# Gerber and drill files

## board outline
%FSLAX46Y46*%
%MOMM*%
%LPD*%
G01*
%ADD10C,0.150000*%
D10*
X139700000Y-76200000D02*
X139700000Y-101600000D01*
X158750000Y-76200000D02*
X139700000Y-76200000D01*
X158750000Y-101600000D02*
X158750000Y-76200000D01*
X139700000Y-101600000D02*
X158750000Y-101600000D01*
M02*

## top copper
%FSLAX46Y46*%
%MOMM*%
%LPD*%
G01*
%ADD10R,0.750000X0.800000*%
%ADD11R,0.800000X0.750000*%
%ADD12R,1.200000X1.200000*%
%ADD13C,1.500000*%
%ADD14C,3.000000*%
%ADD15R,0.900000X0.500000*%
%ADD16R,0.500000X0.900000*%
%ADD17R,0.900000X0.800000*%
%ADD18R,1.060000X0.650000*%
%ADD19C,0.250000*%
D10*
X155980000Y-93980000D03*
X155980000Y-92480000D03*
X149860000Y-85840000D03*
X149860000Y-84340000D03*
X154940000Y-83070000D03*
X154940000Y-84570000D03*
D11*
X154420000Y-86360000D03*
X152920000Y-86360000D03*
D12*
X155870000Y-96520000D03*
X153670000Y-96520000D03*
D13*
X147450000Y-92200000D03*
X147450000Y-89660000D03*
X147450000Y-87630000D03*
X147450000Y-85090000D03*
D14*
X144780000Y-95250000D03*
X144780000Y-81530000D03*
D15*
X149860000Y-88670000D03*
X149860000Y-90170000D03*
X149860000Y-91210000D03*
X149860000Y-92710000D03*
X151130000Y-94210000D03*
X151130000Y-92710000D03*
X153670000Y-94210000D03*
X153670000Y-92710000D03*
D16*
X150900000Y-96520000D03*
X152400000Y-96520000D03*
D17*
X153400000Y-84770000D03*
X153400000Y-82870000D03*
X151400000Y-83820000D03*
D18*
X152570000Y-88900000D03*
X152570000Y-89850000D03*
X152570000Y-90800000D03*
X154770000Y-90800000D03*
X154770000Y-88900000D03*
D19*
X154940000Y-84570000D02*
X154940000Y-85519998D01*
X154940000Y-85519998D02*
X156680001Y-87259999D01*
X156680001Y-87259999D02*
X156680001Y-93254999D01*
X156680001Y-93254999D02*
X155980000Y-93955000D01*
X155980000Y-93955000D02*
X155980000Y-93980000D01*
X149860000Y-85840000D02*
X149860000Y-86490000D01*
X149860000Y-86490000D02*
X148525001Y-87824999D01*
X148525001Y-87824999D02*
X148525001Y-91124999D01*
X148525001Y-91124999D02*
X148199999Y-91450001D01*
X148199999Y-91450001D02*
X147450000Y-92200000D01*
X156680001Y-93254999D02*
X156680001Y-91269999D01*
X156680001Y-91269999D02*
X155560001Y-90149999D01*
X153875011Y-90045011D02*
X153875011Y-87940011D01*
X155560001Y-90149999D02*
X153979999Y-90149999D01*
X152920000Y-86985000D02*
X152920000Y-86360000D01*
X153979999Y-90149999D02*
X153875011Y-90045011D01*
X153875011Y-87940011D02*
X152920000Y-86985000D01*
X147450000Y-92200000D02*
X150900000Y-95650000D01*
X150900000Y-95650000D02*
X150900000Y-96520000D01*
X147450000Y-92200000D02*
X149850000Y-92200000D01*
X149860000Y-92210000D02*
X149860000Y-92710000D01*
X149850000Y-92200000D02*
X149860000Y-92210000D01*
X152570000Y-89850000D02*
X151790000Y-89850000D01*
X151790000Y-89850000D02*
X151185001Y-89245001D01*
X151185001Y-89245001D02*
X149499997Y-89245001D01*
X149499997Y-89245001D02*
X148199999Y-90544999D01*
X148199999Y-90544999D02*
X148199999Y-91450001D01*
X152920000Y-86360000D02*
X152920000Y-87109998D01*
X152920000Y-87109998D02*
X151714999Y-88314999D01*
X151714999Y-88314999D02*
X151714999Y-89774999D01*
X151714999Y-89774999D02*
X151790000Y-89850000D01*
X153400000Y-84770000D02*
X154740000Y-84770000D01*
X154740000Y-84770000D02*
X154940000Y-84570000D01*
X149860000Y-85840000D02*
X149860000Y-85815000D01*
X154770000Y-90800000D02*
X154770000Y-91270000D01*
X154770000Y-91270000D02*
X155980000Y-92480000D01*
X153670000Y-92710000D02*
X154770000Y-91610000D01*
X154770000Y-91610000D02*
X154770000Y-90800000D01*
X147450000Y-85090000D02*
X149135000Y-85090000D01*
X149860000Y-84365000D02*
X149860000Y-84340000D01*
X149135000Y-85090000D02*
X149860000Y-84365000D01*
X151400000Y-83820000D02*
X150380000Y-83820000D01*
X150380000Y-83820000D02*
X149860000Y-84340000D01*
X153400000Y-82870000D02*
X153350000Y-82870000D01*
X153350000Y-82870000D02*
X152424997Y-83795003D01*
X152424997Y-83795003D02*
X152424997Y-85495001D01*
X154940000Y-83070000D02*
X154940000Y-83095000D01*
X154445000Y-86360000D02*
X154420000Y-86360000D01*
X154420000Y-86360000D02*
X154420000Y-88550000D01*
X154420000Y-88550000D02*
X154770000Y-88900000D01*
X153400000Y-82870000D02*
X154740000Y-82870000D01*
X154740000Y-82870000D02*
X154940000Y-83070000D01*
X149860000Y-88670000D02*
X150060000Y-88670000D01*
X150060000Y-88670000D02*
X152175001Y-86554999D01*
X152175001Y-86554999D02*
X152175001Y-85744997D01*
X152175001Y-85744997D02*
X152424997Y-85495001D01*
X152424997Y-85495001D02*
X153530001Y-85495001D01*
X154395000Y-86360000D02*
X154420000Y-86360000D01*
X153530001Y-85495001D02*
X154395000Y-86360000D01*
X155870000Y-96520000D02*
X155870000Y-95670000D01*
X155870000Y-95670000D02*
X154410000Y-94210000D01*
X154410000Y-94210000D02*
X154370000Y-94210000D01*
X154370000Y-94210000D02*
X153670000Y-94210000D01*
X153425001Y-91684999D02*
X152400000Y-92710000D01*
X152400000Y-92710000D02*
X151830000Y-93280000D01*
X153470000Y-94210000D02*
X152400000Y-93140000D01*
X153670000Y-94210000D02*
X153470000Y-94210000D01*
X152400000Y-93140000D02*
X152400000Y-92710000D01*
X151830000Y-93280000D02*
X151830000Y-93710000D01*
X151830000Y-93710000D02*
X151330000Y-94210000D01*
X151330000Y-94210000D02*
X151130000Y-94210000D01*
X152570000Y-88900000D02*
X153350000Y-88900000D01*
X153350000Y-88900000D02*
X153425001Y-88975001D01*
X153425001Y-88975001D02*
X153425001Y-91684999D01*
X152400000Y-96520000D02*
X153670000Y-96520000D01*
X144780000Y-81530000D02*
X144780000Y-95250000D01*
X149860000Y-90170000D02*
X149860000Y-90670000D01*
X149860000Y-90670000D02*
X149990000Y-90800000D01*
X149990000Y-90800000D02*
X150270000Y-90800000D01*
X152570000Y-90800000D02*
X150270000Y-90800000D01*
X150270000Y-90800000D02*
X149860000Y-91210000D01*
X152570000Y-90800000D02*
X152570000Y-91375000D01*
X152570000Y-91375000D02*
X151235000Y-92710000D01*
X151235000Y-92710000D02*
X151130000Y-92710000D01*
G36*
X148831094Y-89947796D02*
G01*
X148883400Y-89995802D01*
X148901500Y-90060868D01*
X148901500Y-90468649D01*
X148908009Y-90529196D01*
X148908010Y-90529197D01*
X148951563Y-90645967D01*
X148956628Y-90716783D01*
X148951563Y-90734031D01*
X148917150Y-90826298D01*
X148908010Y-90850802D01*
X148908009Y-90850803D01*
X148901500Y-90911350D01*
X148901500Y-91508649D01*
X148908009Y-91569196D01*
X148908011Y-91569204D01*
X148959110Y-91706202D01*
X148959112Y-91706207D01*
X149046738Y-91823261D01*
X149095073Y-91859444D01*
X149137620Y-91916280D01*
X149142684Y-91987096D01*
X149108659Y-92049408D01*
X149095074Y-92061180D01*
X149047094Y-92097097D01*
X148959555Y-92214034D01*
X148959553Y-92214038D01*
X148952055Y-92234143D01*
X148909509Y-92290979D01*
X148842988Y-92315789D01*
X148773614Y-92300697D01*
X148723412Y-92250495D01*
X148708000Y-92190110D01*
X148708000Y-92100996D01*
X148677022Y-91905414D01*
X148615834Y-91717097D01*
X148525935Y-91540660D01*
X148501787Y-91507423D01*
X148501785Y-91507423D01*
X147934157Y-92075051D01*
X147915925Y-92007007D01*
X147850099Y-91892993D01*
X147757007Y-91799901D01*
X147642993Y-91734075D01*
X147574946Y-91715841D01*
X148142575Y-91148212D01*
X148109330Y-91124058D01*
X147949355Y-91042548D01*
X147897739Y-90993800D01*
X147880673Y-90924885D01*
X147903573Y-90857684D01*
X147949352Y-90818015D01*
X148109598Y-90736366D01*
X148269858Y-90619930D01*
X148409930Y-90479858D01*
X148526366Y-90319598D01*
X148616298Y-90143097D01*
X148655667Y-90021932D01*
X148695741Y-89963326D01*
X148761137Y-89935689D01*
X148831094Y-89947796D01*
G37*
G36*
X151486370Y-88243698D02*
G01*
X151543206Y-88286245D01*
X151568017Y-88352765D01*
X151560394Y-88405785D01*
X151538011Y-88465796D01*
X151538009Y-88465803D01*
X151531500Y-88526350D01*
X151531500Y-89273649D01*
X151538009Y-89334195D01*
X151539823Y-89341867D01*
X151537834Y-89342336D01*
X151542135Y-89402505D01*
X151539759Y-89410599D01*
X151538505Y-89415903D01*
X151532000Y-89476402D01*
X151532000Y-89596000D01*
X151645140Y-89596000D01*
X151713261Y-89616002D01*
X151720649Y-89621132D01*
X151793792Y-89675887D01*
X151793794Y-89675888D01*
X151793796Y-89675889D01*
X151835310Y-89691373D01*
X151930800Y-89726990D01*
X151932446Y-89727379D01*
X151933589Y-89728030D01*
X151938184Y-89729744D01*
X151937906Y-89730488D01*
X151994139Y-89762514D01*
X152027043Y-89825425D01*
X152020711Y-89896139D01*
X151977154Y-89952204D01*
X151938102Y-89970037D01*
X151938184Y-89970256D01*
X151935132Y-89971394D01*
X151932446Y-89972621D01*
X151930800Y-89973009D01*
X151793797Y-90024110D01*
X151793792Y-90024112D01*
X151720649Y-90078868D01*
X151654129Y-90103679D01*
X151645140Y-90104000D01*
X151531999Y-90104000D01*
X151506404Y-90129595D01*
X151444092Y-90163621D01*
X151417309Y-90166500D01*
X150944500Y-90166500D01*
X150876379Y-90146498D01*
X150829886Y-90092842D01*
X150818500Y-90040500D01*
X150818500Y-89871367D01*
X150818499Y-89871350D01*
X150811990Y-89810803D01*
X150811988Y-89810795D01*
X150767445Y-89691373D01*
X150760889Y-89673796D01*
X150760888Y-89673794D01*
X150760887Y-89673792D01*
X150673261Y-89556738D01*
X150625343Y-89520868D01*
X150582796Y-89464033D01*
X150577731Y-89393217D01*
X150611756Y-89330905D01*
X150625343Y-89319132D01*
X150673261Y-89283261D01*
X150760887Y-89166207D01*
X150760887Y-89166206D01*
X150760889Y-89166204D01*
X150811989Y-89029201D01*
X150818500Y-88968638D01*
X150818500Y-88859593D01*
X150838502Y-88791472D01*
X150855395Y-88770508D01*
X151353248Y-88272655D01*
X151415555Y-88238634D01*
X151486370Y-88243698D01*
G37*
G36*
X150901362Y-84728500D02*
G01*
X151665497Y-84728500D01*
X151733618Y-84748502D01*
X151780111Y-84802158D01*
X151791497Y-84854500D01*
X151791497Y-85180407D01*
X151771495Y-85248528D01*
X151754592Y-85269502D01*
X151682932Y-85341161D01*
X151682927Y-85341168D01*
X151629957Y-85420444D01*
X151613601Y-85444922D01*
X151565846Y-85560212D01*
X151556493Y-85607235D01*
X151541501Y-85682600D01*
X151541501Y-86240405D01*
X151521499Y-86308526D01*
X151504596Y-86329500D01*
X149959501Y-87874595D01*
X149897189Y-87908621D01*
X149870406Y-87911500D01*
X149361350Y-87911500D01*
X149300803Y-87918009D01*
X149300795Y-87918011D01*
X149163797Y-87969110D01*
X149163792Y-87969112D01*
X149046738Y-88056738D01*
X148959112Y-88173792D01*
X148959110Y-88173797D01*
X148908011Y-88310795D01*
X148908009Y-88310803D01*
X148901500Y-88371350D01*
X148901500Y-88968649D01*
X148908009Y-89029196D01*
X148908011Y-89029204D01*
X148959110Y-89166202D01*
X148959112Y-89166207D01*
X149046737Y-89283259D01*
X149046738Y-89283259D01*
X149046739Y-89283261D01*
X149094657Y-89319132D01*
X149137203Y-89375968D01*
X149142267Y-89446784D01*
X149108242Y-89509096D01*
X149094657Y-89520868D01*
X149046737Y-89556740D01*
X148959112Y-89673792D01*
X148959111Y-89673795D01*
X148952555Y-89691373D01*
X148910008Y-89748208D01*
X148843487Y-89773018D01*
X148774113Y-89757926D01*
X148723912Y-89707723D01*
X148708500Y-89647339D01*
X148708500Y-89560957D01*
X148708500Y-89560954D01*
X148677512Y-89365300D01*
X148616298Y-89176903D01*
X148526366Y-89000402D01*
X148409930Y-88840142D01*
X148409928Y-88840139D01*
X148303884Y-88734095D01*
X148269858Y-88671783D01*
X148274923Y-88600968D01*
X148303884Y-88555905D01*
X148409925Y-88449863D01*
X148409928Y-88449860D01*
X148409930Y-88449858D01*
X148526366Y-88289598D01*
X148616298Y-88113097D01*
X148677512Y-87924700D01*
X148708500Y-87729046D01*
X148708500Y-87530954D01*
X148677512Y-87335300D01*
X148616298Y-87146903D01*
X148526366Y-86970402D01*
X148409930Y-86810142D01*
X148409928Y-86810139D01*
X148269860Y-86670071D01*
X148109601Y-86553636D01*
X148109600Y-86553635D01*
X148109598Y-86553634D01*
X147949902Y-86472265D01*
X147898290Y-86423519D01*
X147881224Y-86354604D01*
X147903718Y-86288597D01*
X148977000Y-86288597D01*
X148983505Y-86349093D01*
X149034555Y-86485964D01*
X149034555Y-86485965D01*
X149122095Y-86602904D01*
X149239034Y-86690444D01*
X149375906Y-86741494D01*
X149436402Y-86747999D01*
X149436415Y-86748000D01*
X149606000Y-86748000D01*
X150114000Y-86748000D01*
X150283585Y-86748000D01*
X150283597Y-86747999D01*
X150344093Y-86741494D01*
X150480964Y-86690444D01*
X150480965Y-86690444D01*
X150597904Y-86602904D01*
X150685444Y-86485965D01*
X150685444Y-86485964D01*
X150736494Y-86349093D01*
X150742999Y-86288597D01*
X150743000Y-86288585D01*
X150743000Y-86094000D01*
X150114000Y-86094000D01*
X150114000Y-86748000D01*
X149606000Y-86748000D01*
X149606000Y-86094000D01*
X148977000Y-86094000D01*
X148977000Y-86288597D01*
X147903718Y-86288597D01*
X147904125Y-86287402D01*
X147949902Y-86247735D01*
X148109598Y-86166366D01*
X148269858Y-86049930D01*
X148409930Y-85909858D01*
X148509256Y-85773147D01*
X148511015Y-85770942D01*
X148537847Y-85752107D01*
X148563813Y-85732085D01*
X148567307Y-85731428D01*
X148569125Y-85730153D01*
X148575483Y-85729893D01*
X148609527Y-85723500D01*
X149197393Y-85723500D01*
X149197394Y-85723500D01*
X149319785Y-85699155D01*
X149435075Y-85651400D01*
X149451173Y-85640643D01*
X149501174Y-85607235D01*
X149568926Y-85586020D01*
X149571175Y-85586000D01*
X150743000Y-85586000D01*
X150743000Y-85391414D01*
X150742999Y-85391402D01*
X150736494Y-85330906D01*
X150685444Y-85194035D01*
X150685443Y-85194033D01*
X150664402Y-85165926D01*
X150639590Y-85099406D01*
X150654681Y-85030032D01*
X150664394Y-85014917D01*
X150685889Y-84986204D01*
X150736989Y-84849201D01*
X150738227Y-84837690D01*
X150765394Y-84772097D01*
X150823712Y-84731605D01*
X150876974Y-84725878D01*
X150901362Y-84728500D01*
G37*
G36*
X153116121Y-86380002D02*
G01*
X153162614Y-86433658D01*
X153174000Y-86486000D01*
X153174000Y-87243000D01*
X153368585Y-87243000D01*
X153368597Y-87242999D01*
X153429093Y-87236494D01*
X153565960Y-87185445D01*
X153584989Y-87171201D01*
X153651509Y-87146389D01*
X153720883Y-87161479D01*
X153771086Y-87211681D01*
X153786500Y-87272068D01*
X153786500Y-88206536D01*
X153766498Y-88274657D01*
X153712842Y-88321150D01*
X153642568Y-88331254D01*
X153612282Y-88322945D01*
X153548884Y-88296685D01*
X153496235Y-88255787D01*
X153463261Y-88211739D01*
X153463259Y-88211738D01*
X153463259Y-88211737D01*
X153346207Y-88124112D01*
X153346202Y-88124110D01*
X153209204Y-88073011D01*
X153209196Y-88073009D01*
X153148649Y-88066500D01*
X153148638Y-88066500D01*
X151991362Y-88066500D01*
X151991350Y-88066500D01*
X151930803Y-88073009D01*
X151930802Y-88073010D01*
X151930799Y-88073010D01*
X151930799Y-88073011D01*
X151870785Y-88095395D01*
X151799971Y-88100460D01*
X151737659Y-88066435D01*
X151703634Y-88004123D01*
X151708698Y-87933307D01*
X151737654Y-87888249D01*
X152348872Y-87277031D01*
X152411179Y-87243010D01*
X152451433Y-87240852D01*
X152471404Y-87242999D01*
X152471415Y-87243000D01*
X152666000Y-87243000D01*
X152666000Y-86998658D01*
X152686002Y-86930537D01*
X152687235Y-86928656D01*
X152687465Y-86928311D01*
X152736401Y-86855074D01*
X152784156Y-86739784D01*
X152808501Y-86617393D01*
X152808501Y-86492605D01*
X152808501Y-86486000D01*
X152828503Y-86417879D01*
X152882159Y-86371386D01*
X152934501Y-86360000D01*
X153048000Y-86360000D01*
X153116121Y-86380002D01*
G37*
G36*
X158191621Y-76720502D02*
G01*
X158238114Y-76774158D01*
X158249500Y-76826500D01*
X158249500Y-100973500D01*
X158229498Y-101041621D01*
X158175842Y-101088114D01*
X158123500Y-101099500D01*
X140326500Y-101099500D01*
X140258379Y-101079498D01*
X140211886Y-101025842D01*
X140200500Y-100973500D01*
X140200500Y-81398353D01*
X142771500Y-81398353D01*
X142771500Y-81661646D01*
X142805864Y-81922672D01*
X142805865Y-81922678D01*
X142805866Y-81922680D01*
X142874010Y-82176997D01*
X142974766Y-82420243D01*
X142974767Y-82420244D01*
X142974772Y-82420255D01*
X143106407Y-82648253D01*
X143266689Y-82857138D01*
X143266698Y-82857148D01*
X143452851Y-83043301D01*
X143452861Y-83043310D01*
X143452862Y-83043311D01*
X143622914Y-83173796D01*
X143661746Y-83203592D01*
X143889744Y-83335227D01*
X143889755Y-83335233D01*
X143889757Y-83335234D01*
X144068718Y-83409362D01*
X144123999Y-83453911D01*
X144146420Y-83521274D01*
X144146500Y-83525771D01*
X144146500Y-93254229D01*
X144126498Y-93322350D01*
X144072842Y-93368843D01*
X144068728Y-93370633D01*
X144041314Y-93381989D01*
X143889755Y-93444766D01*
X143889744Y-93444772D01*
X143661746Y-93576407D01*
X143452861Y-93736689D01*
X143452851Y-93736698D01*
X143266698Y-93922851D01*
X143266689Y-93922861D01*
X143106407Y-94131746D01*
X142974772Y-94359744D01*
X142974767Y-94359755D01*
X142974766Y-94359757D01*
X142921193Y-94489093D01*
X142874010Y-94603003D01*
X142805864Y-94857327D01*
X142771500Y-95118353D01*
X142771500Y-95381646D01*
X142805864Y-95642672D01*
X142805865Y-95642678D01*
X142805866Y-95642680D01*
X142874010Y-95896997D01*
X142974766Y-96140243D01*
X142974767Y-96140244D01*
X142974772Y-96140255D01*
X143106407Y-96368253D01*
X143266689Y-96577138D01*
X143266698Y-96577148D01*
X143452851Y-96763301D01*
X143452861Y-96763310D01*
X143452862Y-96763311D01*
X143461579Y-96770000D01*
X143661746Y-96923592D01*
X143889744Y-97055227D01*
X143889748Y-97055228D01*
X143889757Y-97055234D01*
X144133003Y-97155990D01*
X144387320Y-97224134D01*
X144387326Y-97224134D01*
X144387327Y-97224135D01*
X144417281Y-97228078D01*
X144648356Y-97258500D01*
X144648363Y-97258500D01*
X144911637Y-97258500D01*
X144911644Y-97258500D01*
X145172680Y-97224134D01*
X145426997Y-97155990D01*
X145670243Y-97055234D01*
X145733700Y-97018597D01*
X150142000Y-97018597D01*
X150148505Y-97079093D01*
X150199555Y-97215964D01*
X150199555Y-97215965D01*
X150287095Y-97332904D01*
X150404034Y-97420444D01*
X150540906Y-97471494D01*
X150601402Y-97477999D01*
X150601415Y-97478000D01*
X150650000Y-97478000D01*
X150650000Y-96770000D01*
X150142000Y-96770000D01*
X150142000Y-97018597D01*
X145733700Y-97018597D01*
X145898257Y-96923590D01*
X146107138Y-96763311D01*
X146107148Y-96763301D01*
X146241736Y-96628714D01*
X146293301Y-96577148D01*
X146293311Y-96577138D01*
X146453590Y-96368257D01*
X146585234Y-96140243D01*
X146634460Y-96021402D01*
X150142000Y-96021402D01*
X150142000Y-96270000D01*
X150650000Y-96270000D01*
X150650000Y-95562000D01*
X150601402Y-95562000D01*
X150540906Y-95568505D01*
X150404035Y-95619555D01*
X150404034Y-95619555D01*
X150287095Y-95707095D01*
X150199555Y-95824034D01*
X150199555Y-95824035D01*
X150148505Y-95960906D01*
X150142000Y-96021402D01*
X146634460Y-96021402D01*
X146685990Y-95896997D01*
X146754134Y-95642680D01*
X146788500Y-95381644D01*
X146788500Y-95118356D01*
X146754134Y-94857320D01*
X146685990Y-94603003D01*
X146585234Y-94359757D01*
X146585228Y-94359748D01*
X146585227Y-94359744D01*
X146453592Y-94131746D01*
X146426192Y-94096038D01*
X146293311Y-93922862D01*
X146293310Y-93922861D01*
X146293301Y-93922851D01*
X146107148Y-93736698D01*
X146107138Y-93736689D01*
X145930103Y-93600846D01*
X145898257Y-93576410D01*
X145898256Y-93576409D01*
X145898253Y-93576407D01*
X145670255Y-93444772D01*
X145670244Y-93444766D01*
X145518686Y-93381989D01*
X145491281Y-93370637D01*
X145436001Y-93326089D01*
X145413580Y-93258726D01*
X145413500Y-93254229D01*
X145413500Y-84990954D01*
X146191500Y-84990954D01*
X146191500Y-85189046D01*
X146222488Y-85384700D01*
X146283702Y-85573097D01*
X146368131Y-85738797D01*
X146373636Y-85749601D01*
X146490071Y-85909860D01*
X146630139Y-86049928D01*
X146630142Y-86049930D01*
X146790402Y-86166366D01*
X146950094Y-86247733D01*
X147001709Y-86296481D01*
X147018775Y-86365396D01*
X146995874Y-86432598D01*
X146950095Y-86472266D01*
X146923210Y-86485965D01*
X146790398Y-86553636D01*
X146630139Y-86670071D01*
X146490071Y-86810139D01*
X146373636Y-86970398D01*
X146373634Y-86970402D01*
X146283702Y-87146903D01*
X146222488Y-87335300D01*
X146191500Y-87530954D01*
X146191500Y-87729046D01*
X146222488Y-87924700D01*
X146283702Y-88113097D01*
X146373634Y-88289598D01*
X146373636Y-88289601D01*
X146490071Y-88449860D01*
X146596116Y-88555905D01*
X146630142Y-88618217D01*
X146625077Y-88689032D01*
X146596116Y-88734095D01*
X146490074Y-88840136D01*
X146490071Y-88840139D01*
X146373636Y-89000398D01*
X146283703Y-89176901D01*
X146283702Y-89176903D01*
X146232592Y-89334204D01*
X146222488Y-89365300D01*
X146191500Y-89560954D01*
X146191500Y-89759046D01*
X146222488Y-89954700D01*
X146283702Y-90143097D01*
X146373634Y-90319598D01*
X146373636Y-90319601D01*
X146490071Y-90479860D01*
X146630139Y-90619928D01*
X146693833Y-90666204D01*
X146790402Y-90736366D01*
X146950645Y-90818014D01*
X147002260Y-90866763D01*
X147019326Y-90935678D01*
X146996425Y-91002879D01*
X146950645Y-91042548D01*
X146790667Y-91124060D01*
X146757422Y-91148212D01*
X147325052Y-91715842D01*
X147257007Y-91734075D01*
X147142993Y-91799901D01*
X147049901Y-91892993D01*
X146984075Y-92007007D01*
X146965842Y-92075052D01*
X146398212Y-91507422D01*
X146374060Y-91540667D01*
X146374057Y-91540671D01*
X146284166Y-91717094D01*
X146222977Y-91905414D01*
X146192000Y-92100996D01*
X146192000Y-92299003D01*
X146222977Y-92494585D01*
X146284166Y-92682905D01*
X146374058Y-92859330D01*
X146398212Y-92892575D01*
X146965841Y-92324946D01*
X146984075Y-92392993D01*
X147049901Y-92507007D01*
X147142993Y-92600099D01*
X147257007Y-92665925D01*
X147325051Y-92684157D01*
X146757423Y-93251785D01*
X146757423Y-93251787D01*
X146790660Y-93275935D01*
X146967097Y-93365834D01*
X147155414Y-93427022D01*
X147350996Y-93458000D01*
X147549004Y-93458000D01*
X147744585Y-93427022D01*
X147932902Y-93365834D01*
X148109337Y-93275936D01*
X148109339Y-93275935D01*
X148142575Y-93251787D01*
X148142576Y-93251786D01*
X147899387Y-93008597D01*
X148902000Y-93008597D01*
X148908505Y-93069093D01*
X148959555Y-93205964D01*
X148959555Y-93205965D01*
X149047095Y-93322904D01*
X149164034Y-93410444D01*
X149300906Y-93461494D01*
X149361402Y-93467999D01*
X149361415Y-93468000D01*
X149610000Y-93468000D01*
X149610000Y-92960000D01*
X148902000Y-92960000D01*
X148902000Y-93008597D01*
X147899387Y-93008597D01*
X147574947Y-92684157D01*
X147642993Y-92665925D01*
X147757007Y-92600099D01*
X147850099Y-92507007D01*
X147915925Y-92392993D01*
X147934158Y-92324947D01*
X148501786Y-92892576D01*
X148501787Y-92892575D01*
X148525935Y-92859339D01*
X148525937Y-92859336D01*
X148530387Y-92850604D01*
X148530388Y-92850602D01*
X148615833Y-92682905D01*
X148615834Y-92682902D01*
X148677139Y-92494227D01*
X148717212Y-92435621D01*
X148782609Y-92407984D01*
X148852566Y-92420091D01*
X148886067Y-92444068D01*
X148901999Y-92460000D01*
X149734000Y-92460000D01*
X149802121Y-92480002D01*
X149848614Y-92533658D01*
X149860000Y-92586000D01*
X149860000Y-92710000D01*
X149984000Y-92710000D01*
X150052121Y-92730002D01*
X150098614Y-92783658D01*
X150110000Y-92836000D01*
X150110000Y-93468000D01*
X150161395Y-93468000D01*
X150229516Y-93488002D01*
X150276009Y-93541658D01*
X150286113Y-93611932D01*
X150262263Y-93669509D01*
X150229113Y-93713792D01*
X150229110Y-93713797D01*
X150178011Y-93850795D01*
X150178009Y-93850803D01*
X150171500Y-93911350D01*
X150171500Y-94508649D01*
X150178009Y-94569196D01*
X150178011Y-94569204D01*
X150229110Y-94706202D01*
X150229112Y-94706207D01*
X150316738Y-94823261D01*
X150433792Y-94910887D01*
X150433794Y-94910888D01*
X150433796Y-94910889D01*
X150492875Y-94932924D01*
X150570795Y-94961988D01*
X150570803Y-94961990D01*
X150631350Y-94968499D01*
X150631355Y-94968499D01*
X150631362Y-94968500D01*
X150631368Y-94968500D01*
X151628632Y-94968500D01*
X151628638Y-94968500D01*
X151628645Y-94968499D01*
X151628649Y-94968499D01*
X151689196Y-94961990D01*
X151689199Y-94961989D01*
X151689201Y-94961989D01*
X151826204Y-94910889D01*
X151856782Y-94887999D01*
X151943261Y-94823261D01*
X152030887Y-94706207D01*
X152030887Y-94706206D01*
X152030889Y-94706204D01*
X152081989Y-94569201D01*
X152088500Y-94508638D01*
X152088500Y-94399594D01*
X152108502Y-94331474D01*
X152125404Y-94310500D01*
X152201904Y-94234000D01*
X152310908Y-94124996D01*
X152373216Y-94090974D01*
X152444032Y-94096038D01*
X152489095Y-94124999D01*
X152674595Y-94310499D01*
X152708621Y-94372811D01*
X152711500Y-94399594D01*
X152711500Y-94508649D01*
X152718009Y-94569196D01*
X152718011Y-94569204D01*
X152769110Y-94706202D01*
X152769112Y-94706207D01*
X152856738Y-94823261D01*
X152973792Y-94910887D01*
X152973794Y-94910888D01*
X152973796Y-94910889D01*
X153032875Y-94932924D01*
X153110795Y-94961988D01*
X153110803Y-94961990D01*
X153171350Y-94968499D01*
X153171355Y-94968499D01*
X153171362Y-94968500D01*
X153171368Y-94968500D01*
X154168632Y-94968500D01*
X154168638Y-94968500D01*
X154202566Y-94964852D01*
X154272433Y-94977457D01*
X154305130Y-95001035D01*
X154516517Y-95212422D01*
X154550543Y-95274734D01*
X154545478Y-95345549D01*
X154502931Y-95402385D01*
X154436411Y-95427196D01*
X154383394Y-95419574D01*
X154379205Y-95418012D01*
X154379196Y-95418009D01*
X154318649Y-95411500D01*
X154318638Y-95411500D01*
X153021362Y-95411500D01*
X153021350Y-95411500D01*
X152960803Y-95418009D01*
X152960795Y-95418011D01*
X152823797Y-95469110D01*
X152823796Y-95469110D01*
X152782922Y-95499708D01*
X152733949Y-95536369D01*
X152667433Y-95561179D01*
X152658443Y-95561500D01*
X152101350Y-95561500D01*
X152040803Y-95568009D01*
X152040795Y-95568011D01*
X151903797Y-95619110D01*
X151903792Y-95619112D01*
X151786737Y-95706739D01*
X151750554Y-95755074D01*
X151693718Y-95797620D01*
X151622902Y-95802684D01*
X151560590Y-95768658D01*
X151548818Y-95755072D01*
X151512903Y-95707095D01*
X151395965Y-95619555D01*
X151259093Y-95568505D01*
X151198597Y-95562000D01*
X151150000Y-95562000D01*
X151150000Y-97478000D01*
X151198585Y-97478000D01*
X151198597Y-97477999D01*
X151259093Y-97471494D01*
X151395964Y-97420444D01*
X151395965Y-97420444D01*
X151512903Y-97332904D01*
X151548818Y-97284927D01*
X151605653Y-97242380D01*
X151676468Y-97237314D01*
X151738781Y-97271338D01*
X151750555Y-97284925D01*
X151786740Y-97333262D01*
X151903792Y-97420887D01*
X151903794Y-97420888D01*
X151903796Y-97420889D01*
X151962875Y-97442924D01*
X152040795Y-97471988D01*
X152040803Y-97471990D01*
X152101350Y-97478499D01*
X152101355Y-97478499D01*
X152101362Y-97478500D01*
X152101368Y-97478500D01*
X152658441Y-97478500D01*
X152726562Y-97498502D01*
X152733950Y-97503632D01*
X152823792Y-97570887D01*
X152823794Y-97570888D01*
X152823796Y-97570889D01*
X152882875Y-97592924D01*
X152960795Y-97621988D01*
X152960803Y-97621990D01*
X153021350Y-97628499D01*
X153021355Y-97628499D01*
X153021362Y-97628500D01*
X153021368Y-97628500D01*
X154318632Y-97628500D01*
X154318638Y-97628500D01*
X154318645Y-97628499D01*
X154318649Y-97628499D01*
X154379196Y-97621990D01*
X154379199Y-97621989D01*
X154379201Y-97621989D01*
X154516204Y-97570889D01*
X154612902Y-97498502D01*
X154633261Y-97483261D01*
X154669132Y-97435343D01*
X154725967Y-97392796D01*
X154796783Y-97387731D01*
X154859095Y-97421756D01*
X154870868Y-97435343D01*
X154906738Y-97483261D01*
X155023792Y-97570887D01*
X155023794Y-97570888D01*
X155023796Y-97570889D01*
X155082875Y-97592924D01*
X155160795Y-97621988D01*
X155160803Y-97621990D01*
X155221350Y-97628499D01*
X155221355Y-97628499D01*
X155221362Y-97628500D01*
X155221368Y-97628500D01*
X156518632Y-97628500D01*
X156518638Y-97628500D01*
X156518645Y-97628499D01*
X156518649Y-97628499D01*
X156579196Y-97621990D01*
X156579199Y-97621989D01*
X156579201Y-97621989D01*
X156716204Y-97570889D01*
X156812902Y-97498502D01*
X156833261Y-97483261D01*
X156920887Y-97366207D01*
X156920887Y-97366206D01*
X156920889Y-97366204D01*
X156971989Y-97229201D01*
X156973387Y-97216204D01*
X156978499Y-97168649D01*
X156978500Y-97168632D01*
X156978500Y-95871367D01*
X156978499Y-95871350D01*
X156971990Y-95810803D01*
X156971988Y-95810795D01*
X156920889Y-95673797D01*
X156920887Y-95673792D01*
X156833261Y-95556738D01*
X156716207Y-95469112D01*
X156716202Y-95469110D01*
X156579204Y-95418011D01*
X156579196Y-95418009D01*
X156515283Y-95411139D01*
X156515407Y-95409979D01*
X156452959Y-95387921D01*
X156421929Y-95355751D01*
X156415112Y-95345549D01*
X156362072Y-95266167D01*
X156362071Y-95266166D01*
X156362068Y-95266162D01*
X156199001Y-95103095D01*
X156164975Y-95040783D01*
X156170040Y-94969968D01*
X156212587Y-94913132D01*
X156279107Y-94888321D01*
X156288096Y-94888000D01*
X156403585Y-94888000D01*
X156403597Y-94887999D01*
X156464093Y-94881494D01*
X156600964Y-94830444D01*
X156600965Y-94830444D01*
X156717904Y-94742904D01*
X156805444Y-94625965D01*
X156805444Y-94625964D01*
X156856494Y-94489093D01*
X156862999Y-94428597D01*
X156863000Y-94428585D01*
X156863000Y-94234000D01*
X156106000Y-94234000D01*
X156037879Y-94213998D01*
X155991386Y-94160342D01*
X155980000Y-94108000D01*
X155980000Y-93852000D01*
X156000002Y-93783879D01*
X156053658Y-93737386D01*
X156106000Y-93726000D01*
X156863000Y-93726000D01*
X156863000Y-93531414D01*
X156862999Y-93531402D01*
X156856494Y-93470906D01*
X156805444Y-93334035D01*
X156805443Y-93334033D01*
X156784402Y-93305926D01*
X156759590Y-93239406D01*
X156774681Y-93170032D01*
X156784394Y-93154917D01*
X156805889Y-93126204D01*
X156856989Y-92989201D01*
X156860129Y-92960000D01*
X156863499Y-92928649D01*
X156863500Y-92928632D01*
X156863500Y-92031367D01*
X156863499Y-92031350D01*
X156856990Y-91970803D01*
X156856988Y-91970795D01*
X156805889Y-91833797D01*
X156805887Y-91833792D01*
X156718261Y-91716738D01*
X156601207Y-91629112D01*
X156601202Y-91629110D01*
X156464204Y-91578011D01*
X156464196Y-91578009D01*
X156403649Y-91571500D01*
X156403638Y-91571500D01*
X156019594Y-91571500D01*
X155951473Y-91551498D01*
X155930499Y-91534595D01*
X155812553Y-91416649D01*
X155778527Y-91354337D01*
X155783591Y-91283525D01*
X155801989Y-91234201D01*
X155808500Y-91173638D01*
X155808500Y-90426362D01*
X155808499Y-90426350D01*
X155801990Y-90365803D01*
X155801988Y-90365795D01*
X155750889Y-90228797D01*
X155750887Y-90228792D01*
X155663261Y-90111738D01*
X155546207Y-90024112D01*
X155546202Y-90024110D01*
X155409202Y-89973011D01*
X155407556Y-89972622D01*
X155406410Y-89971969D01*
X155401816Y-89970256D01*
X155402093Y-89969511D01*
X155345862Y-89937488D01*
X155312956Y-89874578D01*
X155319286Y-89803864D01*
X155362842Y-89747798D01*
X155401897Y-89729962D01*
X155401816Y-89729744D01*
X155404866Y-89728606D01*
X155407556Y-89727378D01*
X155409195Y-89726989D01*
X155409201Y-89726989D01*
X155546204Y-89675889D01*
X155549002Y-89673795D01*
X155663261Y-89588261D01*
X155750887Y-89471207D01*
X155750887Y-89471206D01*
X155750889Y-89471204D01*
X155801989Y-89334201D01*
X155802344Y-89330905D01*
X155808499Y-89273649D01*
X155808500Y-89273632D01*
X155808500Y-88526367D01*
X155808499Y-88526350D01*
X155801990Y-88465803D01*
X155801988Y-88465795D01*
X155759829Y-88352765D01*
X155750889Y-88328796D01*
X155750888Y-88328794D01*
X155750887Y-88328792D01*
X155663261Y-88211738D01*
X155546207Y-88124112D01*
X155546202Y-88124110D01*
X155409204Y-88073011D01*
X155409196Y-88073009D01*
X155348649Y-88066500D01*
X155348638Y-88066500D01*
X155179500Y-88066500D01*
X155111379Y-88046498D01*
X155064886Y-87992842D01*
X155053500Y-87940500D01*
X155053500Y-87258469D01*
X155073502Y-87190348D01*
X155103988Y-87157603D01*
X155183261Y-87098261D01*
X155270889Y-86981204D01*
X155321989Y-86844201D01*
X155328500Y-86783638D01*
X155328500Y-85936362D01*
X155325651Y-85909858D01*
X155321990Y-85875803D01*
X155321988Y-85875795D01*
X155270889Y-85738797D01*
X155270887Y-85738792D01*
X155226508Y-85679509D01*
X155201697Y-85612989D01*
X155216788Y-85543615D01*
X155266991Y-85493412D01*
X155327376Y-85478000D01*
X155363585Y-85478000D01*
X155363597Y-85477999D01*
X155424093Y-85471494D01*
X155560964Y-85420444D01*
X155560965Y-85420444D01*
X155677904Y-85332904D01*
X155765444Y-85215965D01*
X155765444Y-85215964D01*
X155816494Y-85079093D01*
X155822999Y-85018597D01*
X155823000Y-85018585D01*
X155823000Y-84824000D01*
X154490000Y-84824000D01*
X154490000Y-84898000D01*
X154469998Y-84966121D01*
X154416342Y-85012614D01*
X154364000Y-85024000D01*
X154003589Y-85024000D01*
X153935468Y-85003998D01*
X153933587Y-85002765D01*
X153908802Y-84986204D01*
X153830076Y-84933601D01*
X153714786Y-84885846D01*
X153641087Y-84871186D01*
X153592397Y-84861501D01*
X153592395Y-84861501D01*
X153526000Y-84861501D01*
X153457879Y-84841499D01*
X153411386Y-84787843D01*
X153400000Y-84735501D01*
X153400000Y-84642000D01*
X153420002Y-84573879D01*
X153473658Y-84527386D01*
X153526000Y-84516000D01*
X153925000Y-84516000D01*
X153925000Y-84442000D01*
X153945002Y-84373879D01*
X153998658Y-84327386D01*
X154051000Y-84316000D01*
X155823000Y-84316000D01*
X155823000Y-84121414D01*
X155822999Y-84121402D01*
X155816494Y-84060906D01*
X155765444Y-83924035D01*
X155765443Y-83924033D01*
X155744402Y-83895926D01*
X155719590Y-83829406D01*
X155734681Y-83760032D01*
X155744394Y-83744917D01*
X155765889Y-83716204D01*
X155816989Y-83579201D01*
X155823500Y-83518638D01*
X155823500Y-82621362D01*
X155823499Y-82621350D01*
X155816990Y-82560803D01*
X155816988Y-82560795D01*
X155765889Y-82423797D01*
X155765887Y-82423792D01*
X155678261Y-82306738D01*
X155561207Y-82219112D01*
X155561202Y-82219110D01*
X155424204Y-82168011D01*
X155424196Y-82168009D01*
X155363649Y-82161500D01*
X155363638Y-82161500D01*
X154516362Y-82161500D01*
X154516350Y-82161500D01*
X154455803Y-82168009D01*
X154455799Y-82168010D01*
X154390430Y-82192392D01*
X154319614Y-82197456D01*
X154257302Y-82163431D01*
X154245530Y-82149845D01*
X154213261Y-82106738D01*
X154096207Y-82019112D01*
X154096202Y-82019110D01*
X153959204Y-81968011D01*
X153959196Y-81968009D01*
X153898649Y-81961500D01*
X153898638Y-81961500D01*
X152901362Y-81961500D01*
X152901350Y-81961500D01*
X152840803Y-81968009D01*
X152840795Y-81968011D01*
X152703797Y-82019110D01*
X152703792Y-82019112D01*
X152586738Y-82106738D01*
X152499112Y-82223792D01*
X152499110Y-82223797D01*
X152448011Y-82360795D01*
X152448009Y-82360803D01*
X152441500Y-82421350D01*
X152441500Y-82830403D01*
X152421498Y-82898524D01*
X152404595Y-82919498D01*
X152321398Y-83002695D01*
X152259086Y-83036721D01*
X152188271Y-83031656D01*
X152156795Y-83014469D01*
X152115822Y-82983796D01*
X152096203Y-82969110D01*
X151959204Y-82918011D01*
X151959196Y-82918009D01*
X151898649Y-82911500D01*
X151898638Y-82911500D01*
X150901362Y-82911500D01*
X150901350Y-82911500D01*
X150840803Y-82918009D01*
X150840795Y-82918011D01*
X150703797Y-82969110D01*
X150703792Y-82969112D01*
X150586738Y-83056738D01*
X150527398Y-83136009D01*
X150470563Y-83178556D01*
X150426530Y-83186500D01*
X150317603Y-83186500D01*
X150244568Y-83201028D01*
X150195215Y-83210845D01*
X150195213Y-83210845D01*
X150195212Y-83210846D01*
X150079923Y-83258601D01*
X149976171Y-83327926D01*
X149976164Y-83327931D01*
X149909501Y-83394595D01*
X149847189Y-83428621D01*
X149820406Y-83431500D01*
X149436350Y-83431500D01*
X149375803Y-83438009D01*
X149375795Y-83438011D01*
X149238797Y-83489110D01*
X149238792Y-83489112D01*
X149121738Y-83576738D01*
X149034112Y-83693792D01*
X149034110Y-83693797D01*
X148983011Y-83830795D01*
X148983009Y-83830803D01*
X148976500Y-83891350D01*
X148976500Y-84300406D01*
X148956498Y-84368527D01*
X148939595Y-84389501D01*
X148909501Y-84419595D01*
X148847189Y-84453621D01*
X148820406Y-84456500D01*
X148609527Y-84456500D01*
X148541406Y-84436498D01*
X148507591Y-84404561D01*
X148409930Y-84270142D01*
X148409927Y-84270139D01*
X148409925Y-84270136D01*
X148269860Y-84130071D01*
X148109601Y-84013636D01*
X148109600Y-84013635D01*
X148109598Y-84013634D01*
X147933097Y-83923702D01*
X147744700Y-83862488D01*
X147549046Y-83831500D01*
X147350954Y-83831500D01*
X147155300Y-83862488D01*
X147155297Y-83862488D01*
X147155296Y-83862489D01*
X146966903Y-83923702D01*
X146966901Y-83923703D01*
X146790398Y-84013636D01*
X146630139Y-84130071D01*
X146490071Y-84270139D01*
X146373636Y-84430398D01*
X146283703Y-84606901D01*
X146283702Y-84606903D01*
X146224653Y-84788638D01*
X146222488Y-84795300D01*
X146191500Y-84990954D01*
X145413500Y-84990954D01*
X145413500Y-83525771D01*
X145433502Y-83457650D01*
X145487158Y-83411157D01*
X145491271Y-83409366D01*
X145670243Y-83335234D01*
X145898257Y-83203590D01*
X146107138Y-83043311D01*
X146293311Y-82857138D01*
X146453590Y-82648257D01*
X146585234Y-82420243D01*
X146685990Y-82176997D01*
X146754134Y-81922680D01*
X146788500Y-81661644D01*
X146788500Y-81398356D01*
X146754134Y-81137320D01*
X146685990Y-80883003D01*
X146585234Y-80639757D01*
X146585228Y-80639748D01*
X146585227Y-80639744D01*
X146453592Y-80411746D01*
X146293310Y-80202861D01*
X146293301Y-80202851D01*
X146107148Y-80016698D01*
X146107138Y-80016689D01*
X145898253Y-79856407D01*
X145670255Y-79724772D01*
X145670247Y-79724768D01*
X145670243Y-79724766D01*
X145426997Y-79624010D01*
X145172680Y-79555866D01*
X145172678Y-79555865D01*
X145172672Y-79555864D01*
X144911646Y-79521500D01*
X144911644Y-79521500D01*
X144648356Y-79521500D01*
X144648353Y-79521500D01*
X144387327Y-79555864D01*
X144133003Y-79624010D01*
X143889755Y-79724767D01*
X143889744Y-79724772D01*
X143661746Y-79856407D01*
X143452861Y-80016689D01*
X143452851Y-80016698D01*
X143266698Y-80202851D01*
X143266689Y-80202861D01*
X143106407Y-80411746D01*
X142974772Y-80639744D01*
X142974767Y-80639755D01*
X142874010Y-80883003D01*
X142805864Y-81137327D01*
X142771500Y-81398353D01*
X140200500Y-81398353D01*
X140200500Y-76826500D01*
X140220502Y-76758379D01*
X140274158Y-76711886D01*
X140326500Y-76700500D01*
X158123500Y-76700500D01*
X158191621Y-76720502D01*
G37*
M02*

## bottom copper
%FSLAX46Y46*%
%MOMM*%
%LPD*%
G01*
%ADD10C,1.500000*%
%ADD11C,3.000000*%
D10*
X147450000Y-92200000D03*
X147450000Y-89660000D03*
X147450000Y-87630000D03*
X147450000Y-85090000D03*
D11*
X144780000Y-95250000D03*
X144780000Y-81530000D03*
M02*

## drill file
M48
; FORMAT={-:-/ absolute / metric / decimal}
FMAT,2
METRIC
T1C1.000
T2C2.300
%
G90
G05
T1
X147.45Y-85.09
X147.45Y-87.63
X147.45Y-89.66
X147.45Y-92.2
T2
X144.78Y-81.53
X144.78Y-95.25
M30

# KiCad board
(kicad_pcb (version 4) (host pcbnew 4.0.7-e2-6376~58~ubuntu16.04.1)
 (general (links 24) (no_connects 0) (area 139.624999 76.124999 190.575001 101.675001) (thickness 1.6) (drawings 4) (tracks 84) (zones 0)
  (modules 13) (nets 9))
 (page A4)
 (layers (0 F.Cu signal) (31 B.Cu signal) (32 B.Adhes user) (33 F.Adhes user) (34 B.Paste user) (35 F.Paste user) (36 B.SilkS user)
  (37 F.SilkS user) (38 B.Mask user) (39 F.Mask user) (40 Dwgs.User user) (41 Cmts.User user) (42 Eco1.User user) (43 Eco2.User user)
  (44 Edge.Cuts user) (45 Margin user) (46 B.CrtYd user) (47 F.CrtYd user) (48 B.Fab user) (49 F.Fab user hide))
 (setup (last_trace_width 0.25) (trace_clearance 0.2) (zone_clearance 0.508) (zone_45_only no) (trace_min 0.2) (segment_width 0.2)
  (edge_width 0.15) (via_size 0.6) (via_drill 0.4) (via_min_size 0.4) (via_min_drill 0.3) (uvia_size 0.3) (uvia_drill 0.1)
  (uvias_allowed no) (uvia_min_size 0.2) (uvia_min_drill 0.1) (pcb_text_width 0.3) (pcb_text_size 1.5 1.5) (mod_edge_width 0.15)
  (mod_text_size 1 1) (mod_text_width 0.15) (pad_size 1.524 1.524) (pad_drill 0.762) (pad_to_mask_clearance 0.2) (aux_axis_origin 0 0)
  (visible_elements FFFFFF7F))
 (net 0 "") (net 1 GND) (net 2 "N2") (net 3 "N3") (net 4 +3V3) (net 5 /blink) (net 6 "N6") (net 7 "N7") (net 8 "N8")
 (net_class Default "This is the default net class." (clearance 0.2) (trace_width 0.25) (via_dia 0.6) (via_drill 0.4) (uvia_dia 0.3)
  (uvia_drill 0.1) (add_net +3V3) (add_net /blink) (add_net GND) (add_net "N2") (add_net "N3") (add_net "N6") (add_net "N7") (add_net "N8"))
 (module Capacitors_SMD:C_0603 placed (layer F.Cu) (at 155.98 93.23 270)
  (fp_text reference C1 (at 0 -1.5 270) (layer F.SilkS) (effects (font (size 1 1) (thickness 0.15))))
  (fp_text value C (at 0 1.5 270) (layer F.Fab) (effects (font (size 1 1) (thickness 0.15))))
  (pad 2 smd rect (at 0.75 0 270) (size 0.8 0.75) (layers F.Cu F.Paste F.Mask) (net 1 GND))
  (pad 1 smd rect (at -0.75 0 270) (size 0.8 0.75) (layers F.Cu F.Paste F.Mask) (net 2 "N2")))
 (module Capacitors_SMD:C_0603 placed (layer F.Cu) (at 149.86 85.09 270)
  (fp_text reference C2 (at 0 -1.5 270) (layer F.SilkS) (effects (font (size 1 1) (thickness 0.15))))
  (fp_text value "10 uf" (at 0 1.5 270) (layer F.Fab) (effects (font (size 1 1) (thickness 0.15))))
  (pad 2 smd rect (at 0.75 0 270) (size 0.8 0.75) (layers F.Cu F.Paste F.Mask) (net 1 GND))
  (pad 1 smd rect (at -0.75 0 270) (size 0.8 0.75) (layers F.Cu F.Paste F.Mask) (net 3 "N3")))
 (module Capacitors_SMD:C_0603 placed (layer F.Cu) (at 154.94 83.82 90)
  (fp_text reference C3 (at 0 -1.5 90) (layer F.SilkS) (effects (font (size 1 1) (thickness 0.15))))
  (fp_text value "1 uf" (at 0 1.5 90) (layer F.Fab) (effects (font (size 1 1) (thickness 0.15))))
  (pad 2 smd rect (at 0.75 0 90) (size 0.8 0.75) (layers F.Cu F.Paste F.Mask) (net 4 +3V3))
  (pad 1 smd rect (at -0.75 0 90) (size 0.8 0.75) (layers F.Cu F.Paste F.Mask) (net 1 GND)))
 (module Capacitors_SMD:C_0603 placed (layer F.Cu) (at 153.67 86.36)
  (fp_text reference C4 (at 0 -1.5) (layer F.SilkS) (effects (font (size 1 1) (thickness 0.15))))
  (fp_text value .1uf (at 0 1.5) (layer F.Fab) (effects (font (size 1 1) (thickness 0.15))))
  (pad 2 smd rect (at 0.75 0) (size 0.8 0.75) (layers F.Cu F.Paste F.Mask) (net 4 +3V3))
  (pad 1 smd rect (at -0.75 0) (size 0.8 0.75) (layers F.Cu F.Paste F.Mask) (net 1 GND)))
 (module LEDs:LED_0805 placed (layer F.Cu) (at 154.77 96.52)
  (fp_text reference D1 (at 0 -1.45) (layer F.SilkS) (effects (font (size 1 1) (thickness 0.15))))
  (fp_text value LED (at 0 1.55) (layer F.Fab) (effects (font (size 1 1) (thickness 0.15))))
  (pad 2 smd rect (at 1.1 0 180) (size 1.2 1.2) (layers F.Cu F.Paste F.Mask) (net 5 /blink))
  (pad 1 smd rect (at -1.1 0 180) (size 1.2 1.2) (layers F.Cu F.Paste F.Mask) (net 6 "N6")))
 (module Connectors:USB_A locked (layer F.Cu) (at 147.45 85.09 270)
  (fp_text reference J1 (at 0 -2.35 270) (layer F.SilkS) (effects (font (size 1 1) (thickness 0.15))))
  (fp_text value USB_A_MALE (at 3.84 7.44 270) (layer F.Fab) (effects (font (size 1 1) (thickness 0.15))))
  (pad 4 thru_hole circle (at 7.11 0 180) (size 1.5 1.5) (drill 1) (layers *.Cu *.Mask) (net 1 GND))
  (pad 3 thru_hole circle (at 4.57 0 180) (size 1.5 1.5) (drill 1) (layers *.Cu *.Mask))
  (pad 2 thru_hole circle (at 2.54 0 180) (size 1.5 1.5) (drill 1) (layers *.Cu *.Mask))
  (pad 1 thru_hole circle (at 0 0 180) (size 1.5 1.5) (drill 1) (layers *.Cu *.Mask) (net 3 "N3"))
  (pad 5 thru_hole circle (at 10.16 2.67 180) (size 3 3) (drill 2.3) (layers *.Cu *.Mask) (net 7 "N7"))
  (pad 5 thru_hole circle (at -3.56 2.67 180) (size 3 3) (drill 2.3) (layers *.Cu *.Mask) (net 7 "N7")))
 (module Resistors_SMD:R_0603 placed (layer F.Cu) (at 149.86 89.42 270)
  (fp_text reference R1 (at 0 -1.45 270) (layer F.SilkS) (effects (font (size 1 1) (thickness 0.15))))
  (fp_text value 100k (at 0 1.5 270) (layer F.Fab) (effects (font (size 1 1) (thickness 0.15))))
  (pad 1 smd rect (at -0.75 0 270) (size 0.5 0.9) (layers F.Cu F.Paste F.Mask) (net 4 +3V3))
  (pad 2 smd rect (at 0.75 0 270) (size 0.5 0.9) (layers F.Cu F.Paste F.Mask) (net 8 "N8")))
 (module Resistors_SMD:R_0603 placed (layer F.Cu) (at 149.86 91.96 270)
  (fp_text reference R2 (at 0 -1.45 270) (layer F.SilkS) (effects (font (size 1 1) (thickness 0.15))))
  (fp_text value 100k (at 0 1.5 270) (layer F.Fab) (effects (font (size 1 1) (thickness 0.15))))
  (pad 1 smd rect (at -0.75 0 270) (size 0.5 0.9) (layers F.Cu F.Paste F.Mask) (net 8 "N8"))
  (pad 2 smd rect (at 0.75 0 270) (size 0.5 0.9) (layers F.Cu F.Paste F.Mask) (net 1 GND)))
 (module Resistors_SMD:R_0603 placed (layer F.Cu) (at 151.13 93.46 90)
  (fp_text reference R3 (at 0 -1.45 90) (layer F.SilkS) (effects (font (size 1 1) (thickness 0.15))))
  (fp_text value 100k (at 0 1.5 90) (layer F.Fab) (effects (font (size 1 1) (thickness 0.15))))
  (pad 1 smd rect (at -0.75 0 90) (size 0.5 0.9) (layers F.Cu F.Paste F.Mask) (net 5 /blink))
  (pad 2 smd rect (at 0.75 0 90) (size 0.5 0.9) (layers F.Cu F.Paste F.Mask) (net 8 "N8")))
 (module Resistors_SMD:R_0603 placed (layer F.Cu) (at 153.67 93.46 90)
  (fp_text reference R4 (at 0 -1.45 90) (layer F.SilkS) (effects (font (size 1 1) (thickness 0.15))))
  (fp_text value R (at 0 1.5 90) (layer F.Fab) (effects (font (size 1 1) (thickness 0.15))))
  (pad 1 smd rect (at -0.75 0 90) (size 0.5 0.9) (layers F.Cu F.Paste F.Mask) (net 5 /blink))
  (pad 2 smd rect (at 0.75 0 90) (size 0.5 0.9) (layers F.Cu F.Paste F.Mask) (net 2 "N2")))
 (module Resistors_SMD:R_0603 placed (layer F.Cu) (at 151.65 96.52)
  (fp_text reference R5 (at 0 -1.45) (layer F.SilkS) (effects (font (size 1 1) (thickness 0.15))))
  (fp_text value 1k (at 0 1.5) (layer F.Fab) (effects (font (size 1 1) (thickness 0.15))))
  (pad 1 smd rect (at -0.75 0) (size 0.5 0.9) (layers F.Cu F.Paste F.Mask) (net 1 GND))
  (pad 2 smd rect (at 0.75 0) (size 0.5 0.9) (layers F.Cu F.Paste F.Mask) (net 6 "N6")))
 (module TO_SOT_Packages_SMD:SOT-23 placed (layer F.Cu) (at 152.4 83.82 180)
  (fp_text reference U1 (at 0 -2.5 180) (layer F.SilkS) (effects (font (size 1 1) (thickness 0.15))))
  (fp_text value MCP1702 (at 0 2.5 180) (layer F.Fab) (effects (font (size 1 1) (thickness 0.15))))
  (pad 1 smd rect (at -1 -0.95 180) (size 0.9 0.8) (layers F.Cu F.Paste F.Mask) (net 1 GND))
  (pad 2 smd rect (at -1 0.95 180) (size 0.9 0.8) (layers F.Cu F.Paste F.Mask) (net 4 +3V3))
  (pad 3 smd rect (at 1 0 180) (size 0.9 0.8) (layers F.Cu F.Paste F.Mask) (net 3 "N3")))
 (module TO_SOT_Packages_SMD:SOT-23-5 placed (layer F.Cu) (at 153.67 89.85)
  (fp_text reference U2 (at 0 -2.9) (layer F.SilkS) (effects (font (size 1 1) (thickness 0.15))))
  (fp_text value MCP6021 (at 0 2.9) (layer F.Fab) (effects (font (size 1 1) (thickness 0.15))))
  (pad 1 smd rect (at -1.1 -0.95) (size 1.06 0.65) (layers F.Cu F.Paste F.Mask) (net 5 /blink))
  (pad 2 smd rect (at -1.1 0) (size 1.06 0.65) (layers F.Cu F.Paste F.Mask) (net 1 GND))
  (pad 3 smd rect (at -1.1 0.95) (size 1.06 0.65) (layers F.Cu F.Paste F.Mask) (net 8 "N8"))
  (pad 4 smd rect (at 1.1 0.95) (size 1.06 0.65) (layers F.Cu F.Paste F.Mask) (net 2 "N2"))
  (pad 5 smd rect (at 1.1 -0.95) (size 1.06 0.65) (layers F.Cu F.Paste F.Mask) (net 4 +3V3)))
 (gr_line (start 139.7 76.2) (end 139.7 101.6) (layer Edge.Cuts) (width 0.15))
 (gr_line (start 158.75 76.2) (end 139.7 76.2) (layer Edge.Cuts) (width 0.15))
 (gr_line (start 158.75 101.6) (end 158.75 76.2) (layer Edge.Cuts) (width 0.15))
 (gr_line (start 139.7 101.6) (end 158.75 101.6) (layer Edge.Cuts) (width 0.15))
 (segment (start 154.94 84.57) (end 154.94 85.519998) (width 0.25) (layer F.Cu) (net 1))
 (segment (start 154.94 85.519998) (end 156.680001 87.259999) (width 0.25) (layer F.Cu) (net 1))
 (segment (start 156.680001 87.259999) (end 156.680001 93.254999) (width 0.25) (layer F.Cu) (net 1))
 (segment (start 156.680001 93.254999) (end 155.98 93.955) (width 0.25) (layer F.Cu) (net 1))
 (segment (start 155.98 93.955) (end 155.98 93.98) (width 0.25) (layer F.Cu) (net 1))
 (segment (start 149.86 85.84) (end 149.86 86.49) (width 0.25) (layer F.Cu) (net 1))
 (segment (start 149.86 86.49) (end 148.525001 87.824999) (width 0.25) (layer F.Cu) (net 1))
 (segment (start 148.525001 87.824999) (end 148.525001 91.124999) (width 0.25) (layer F.Cu) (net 1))
 (segment (start 148.525001 91.124999) (end 148.199999 91.450001) (width 0.25) (layer F.Cu) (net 1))
 (segment (start 148.199999 91.450001) (end 147.45 92.2) (width 0.25) (layer F.Cu) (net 1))
 (segment (start 156.680001 93.254999) (end 156.680001 91.269999) (width 0.25) (layer F.Cu) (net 1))
 (segment (start 156.680001 91.269999) (end 155.560001 90.149999) (width 0.25) (layer F.Cu) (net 1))
 (segment (start 153.875011 90.045011) (end 153.875011 87.940011) (width 0.25) (layer F.Cu) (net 1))
 (segment (start 155.560001 90.149999) (end 153.979999 90.149999) (width 0.25) (layer F.Cu) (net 1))
 (segment (start 152.92 86.985) (end 152.92 86.36) (width 0.25) (layer F.Cu) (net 1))
 (segment (start 153.979999 90.149999) (end 153.875011 90.045011) (width 0.25) (layer F.Cu) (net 1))
 (segment (start 153.875011 87.940011) (end 152.92 86.985) (width 0.25) (layer F.Cu) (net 1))
 (segment (start 147.45 92.2) (end 150.9 95.65) (width 0.25) (layer F.Cu) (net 1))
 (segment (start 150.9 95.65) (end 150.9 96.52) (width 0.25) (layer F.Cu) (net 1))
 (segment (start 147.45 92.2) (end 149.85 92.2) (width 0.25) (layer F.Cu) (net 1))
 (segment (start 149.86 92.21) (end 149.86 92.71) (width 0.25) (layer F.Cu) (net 1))
 (segment (start 149.85 92.2) (end 149.86 92.21) (width 0.25) (layer F.Cu) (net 1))
 (segment (start 152.57 89.85) (end 151.79 89.85) (width 0.25) (layer F.Cu) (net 1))
 (segment (start 151.79 89.85) (end 151.185001 89.245001) (width 0.25) (layer F.Cu) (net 1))
 (segment (start 151.185001 89.245001) (end 149.499997 89.245001) (width 0.25) (layer F.Cu) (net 1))
 (segment (start 149.499997 89.245001) (end 148.199999 90.544999) (width 0.25) (layer F.Cu) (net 1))
 (segment (start 148.199999 90.544999) (end 148.199999 91.450001) (width 0.25) (layer F.Cu) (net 1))
 (segment (start 152.92 86.36) (end 152.92 87.109998) (width 0.25) (layer F.Cu) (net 1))
 (segment (start 152.92 87.109998) (end 151.714999 88.314999) (width 0.25) (layer F.Cu) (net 1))
 (segment (start 151.714999 88.314999) (end 151.714999 89.774999) (width 0.25) (layer F.Cu) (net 1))
 (segment (start 151.714999 89.774999) (end 151.79 89.85) (width 0.25) (layer F.Cu) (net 1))
 (segment (start 153.4 84.77) (end 154.74 84.77) (width 0.25) (layer F.Cu) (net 1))
 (segment (start 154.74 84.77) (end 154.94 84.57) (width 0.25) (layer F.Cu) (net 1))
 (segment (start 149.86 85.84) (end 149.86 85.815) (width 0.25) (layer F.Cu) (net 1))
 (segment (start 154.77 90.8) (end 154.77 91.27) (width 0.25) (layer F.Cu) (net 2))
 (segment (start 154.77 91.27) (end 155.98 92.48) (width 0.25) (layer F.Cu) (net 2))
 (segment (start 153.67 92.71) (end 154.77 91.61) (width 0.25) (layer F.Cu) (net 2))
 (segment (start 154.77 91.61) (end 154.77 90.8) (width 0.25) (layer F.Cu) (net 2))
 (segment (start 147.45 85.09) (end 149.135 85.09) (width 0.25) (layer F.Cu) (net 3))
 (segment (start 149.86 84.365) (end 149.86 84.34) (width 0.25) (layer F.Cu) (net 3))
 (segment (start 149.135 85.09) (end 149.86 84.365) (width 0.25) (layer F.Cu) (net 3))
 (segment (start 151.4 83.82) (end 150.38 83.82) (width 0.25) (layer F.Cu) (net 3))
 (segment (start 150.38 83.82) (end 149.86 84.34) (width 0.25) (layer F.Cu) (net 3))
 (segment (start 153.4 82.87) (end 153.35 82.87) (width 0.25) (layer F.Cu) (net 4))
 (segment (start 153.35 82.87) (end 152.424997 83.795003) (width 0.25) (layer F.Cu) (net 4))
 (segment (start 152.424997 83.795003) (end 152.424997 85.495001) (width 0.25) (layer F.Cu) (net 4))
 (segment (start 154.94 83.07) (end 154.94 83.095) (width 0.25) (layer F.Cu) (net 4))
 (segment (start 154.445 86.36) (end 154.42 86.36) (width 0.25) (layer F.Cu) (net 4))
 (segment (start 154.42 86.36) (end 154.42 88.55) (width 0.25) (layer F.Cu) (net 4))
 (segment (start 154.42 88.55) (end 154.77 88.9) (width 0.25) (layer F.Cu) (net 4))
 (segment (start 153.4 82.87) (end 154.74 82.87) (width 0.25) (layer F.Cu) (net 4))
 (segment (start 154.74 82.87) (end 154.94 83.07) (width 0.25) (layer F.Cu) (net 4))
 (segment (start 149.86 88.67) (end 150.06 88.67) (width 0.25) (layer F.Cu) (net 4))
 (segment (start 150.06 88.67) (end 152.175001 86.554999) (width 0.25) (layer F.Cu) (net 4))
 (segment (start 152.175001 86.554999) (end 152.175001 85.744997) (width 0.25) (layer F.Cu) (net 4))
 (segment (start 152.175001 85.744997) (end 152.424997 85.495001) (width 0.25) (layer F.Cu) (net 4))
 (segment (start 152.424997 85.495001) (end 153.530001 85.495001) (width 0.25) (layer F.Cu) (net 4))
 (segment (start 154.395 86.36) (end 154.42 86.36) (width 0.25) (layer F.Cu) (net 4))
 (segment (start 153.530001 85.495001) (end 154.395 86.36) (width 0.25) (layer F.Cu) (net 4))
 (segment (start 155.87 96.52) (end 155.87 95.67) (width 0.25) (layer F.Cu) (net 5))
 (segment (start 155.87 95.67) (end 154.41 94.21) (width 0.25) (layer F.Cu) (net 5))
 (segment (start 154.41 94.21) (end 154.37 94.21) (width 0.25) (layer F.Cu) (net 5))
 (segment (start 154.37 94.21) (end 153.67 94.21) (width 0.25) (layer F.Cu) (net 5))
 (segment (start 153.425001 91.684999) (end 152.4 92.71) (width 0.25) (layer F.Cu) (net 5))
 (segment (start 152.4 92.71) (end 151.83 93.28) (width 0.25) (layer F.Cu) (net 5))
 (segment (start 153.47 94.21) (end 152.4 93.14) (width 0.25) (layer F.Cu) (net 5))
 (segment (start 153.67 94.21) (end 153.47 94.21) (width 0.25) (layer F.Cu) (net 5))
 (segment (start 152.4 93.14) (end 152.4 92.71) (width 0.25) (layer F.Cu) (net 5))
 (segment (start 151.83 93.28) (end 151.83 93.71) (width 0.25) (layer F.Cu) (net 5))
 (segment (start 151.83 93.71) (end 151.33 94.21) (width 0.25) (layer F.Cu) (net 5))
 (segment (start 151.33 94.21) (end 151.13 94.21) (width 0.25) (layer F.Cu) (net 5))
 (segment (start 152.57 88.9) (end 153.35 88.9) (width 0.25) (layer F.Cu) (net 5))
 (segment (start 153.35 88.9) (end 153.425001 88.975001) (width 0.25) (layer F.Cu) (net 5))
 (segment (start 153.425001 88.975001) (end 153.425001 91.684999) (width 0.25) (layer F.Cu) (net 5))
 (segment (start 152.4 96.52) (end 153.67 96.52) (width 0.25) (layer F.Cu) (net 6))
 (segment (start 144.78 81.53) (end 144.78 95.25) (width 0.25) (layer F.Cu) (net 7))
 (segment (start 149.86 90.17) (end 149.86 90.67) (width 0.25) (layer F.Cu) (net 8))
 (segment (start 149.86 90.67) (end 149.99 90.8) (width 0.25) (layer F.Cu) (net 8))
 (segment (start 149.99 90.8) (end 150.27 90.8) (width 0.25) (layer F.Cu) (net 8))
 (segment (start 152.57 90.8) (end 150.27 90.8) (width 0.25) (layer F.Cu) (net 8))
 (segment (start 150.27 90.8) (end 149.86 91.21) (width 0.25) (layer F.Cu) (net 8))
 (segment (start 152.57 90.8) (end 152.57 91.375) (width 0.25) (layer F.Cu) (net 8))
 (segment (start 152.57 91.375) (end 151.235 92.71) (width 0.25) (layer F.Cu) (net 8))
 (segment (start 151.235 92.71) (end 151.13 92.71) (width 0.25) (layer F.Cu) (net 8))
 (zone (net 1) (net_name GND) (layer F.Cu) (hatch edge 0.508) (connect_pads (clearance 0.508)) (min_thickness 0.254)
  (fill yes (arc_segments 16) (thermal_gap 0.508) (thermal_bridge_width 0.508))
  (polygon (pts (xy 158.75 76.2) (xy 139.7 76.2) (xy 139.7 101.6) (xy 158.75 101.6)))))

